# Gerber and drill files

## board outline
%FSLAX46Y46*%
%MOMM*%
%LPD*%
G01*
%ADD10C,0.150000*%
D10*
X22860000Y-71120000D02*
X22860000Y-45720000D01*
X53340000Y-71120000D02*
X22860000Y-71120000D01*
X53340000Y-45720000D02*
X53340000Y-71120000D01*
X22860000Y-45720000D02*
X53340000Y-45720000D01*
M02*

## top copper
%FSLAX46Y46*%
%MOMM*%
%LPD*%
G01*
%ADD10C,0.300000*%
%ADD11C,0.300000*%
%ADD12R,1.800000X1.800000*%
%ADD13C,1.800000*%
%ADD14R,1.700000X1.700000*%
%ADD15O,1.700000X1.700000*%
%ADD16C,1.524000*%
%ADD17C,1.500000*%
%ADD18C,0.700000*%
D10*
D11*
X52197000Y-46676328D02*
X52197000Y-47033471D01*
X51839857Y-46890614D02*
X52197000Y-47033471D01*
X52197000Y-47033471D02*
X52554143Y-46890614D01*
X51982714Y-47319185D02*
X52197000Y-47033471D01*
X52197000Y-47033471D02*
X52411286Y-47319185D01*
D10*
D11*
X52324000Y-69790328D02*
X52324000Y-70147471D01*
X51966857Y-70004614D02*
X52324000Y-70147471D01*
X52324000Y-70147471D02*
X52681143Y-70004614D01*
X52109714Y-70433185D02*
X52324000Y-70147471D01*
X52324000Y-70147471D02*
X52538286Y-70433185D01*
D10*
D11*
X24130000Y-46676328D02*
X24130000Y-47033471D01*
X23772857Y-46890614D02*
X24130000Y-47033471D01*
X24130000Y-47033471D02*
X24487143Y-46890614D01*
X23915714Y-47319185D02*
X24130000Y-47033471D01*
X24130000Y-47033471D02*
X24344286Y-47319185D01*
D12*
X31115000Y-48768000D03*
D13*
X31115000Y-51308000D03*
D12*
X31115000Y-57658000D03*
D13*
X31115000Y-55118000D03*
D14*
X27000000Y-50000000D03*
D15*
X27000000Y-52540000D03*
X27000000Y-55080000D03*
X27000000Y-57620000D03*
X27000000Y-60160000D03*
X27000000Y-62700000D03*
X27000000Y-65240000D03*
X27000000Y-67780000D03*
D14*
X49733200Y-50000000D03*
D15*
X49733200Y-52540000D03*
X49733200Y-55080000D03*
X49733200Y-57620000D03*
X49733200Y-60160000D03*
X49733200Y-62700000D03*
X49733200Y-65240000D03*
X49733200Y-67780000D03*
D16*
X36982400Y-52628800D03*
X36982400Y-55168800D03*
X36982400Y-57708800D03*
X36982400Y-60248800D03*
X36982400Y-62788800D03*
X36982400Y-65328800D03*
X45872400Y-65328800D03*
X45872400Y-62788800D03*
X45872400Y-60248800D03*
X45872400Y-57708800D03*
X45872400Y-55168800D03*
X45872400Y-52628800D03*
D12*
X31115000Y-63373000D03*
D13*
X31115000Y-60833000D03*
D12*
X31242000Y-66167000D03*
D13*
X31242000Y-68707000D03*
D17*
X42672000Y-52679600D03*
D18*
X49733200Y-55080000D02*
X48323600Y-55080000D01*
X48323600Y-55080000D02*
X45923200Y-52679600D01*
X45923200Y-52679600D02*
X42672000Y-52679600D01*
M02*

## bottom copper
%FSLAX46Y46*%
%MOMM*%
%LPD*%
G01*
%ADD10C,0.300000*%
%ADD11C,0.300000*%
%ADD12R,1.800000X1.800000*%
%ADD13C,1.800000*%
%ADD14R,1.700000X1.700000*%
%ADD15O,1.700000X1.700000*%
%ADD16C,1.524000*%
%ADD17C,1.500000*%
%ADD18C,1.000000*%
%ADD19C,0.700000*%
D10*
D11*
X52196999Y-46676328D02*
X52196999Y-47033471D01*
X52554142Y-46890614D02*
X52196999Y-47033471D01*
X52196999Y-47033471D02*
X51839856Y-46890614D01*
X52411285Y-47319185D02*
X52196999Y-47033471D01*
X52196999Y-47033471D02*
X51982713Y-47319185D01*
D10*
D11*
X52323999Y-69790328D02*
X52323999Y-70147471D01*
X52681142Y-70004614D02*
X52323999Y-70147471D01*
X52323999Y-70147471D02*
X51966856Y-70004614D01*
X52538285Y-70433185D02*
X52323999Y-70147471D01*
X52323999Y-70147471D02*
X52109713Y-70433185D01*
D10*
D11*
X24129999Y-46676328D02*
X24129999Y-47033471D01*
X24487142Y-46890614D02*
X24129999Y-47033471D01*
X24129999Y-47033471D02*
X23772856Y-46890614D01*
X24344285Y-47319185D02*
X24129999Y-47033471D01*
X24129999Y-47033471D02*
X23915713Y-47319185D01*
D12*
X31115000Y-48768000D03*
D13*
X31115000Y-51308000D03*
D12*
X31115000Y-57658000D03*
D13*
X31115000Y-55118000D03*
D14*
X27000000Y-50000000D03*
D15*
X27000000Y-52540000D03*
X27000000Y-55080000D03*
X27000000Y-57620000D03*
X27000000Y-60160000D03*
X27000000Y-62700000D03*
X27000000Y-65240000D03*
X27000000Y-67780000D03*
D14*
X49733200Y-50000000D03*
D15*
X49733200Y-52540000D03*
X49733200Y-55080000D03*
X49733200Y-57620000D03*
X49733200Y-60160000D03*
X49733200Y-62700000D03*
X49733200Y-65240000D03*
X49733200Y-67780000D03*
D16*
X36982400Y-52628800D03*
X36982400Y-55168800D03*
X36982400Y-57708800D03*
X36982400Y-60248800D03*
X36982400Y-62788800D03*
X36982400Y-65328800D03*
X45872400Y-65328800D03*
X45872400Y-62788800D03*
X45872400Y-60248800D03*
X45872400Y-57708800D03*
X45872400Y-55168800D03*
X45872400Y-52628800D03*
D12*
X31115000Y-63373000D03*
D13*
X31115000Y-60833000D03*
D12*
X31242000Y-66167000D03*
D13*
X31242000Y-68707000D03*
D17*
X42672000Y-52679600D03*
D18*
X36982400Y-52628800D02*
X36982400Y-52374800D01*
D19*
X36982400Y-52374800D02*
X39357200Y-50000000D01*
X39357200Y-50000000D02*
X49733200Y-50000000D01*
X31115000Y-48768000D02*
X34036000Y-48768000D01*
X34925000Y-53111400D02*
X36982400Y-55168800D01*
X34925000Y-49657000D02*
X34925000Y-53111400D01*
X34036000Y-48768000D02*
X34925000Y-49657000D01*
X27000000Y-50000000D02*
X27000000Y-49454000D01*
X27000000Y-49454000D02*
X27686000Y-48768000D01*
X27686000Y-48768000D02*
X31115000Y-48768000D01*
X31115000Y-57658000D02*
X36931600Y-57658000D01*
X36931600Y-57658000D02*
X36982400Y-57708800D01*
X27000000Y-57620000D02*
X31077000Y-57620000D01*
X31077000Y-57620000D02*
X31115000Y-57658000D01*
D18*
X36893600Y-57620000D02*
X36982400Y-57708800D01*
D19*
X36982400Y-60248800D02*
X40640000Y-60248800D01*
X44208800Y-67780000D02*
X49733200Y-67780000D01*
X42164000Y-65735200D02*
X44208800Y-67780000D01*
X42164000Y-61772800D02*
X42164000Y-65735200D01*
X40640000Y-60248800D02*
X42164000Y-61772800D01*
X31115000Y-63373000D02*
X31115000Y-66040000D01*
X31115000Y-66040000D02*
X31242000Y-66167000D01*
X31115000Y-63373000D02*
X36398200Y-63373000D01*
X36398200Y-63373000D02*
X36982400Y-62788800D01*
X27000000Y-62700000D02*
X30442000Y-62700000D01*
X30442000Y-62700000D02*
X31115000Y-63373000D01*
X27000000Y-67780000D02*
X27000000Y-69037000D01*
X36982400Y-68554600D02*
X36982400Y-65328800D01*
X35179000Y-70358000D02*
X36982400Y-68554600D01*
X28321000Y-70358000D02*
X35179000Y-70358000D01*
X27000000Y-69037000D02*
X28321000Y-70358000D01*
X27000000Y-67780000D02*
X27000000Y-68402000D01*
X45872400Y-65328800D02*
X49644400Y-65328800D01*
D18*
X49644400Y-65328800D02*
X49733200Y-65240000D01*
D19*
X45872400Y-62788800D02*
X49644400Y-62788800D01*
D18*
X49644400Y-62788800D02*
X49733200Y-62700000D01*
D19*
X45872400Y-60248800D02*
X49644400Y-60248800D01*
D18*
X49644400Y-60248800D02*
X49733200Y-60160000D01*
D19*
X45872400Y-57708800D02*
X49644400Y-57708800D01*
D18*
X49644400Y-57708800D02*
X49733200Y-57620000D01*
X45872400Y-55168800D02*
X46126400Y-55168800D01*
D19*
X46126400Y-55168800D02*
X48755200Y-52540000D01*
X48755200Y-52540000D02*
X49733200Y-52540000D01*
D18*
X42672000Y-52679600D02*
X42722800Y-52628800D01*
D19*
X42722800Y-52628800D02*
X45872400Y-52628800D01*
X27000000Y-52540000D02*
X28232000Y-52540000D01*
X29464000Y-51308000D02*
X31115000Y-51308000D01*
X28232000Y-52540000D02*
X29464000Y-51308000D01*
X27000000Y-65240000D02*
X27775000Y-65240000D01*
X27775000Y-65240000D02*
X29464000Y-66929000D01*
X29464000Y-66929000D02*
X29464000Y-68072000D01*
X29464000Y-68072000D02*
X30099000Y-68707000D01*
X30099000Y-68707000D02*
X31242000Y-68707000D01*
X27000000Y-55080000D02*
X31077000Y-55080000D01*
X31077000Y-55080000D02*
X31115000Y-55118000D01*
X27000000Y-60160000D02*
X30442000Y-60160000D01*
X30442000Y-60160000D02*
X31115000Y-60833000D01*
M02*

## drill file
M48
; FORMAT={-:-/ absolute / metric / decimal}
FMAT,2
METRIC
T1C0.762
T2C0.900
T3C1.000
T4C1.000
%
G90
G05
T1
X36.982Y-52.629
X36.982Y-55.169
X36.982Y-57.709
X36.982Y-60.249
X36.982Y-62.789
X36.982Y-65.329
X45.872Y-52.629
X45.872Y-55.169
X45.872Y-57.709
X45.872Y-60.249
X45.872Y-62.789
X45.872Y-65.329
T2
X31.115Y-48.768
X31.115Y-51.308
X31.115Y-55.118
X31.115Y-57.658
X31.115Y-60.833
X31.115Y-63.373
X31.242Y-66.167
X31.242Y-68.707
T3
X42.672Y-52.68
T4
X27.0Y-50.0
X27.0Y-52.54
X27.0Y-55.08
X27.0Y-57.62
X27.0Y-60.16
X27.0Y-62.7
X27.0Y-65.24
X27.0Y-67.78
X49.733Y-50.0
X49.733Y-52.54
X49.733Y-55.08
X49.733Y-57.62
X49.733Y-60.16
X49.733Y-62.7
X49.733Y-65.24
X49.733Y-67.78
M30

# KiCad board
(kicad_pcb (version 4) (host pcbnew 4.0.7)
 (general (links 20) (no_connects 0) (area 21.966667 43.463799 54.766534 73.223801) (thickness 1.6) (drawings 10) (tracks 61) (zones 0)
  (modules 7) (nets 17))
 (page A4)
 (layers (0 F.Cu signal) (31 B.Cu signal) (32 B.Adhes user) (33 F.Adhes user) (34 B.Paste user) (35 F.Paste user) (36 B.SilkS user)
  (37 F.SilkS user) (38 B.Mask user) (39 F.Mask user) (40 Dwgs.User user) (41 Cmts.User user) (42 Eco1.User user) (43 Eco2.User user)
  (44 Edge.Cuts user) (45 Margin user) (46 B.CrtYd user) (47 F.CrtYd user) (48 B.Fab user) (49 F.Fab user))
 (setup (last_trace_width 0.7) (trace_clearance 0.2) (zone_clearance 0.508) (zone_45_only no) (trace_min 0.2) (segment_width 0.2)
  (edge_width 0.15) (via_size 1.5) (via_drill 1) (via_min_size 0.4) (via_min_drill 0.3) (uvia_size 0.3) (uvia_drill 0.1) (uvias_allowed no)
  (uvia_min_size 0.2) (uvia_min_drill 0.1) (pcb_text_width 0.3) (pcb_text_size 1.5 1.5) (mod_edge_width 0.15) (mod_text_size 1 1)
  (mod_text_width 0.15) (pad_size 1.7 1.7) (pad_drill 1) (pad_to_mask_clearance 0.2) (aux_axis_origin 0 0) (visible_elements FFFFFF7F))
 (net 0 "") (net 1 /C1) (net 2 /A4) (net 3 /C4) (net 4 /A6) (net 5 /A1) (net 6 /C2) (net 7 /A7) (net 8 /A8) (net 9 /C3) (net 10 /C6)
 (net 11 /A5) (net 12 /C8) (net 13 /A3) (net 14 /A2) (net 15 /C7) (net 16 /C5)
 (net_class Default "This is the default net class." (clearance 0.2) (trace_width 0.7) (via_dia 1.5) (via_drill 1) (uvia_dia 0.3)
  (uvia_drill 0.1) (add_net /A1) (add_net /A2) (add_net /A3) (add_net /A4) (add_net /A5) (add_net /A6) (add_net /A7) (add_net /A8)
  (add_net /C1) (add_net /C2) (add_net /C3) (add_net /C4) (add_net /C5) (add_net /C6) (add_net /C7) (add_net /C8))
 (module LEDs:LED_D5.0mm (layer F.Cu) (at 31.115 48.768 270)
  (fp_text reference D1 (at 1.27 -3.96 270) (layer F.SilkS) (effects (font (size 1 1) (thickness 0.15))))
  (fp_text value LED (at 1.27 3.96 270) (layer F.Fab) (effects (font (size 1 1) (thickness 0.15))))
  (pad 1 thru_hole rect (at 0 0 270) (size 1.8 1.8) (drill 0.9) (layers *.Cu *.Mask) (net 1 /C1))
  (pad 2 thru_hole circle (at 2.54 0 270) (size 1.8 1.8) (drill 0.9) (layers *.Cu *.Mask) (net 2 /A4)))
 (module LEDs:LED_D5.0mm (layer F.Cu) (at 31.115 57.658 90)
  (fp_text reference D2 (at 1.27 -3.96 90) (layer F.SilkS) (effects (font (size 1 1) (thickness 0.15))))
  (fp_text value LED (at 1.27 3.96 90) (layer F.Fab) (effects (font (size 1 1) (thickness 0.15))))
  (pad 1 thru_hole rect (at 0 0 90) (size 1.8 1.8) (drill 0.9) (layers *.Cu *.Mask) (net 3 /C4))
  (pad 2 thru_hole circle (at 2.54 0 90) (size 1.8 1.8) (drill 0.9) (layers *.Cu *.Mask) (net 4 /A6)))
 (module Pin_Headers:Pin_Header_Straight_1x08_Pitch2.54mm (layer F.Cu) (at 27 50)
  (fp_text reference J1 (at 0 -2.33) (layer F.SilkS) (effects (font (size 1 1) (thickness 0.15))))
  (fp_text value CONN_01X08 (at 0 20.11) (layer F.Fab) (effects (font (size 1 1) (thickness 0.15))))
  (pad 1 thru_hole rect (at 0 0) (size 1.7 1.7) (drill 1) (layers *.Cu *.Mask) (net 1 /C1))
  (pad 2 thru_hole oval (at 0 2.54) (size 1.7 1.7) (drill 1) (layers *.Cu *.Mask) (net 2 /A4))
  (pad 3 thru_hole oval (at 0 5.08) (size 1.7 1.7) (drill 1) (layers *.Cu *.Mask) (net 4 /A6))
  (pad 4 thru_hole oval (at 0 7.62) (size 1.7 1.7) (drill 1) (layers *.Cu *.Mask) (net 3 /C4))
  (pad 5 thru_hole oval (at 0 10.16) (size 1.7 1.7) (drill 1) (layers *.Cu *.Mask) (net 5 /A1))
  (pad 6 thru_hole oval (at 0 12.7) (size 1.7 1.7) (drill 1) (layers *.Cu *.Mask) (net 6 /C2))
  (pad 7 thru_hole oval (at 0 15.24) (size 1.7 1.7) (drill 1) (layers *.Cu *.Mask) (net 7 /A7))
  (pad 8 thru_hole oval (at 0 17.78) (size 1.7 1.7) (drill 1) (layers *.Cu *.Mask) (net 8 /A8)))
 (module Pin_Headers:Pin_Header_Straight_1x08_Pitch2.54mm (layer F.Cu) (at 49.7332 50)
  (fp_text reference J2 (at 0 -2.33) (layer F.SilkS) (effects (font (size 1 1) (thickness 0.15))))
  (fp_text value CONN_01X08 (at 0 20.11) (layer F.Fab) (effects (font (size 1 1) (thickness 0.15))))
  (pad 1 thru_hole rect (at 0 0) (size 1.7 1.7) (drill 1) (layers *.Cu *.Mask) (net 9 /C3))
  (pad 2 thru_hole oval (at 0 2.54) (size 1.7 1.7) (drill 1) (layers *.Cu *.Mask) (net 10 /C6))
  (pad 3 thru_hole oval (at 0 5.08) (size 1.7 1.7) (drill 1) (layers *.Cu *.Mask) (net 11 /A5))
  (pad 4 thru_hole oval (at 0 7.62) (size 1.7 1.7) (drill 1) (layers *.Cu *.Mask) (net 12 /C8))
  (pad 5 thru_hole oval (at 0 10.16) (size 1.7 1.7) (drill 1) (layers *.Cu *.Mask) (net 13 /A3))
  (pad 6 thru_hole oval (at 0 12.7) (size 1.7 1.7) (drill 1) (layers *.Cu *.Mask) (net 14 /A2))
  (pad 7 thru_hole oval (at 0 15.24) (size 1.7 1.7) (drill 1) (layers *.Cu *.Mask) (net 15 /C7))
  (pad 8 thru_hole oval (at 0 17.78) (size 1.7 1.7) (drill 1) (layers *.Cu *.Mask) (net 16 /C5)))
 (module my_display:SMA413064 (layer F.Cu) (at 36.9824 52.6288)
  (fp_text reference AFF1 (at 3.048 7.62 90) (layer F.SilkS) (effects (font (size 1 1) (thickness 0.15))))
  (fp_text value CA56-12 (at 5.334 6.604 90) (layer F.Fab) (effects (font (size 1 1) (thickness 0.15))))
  (pad 1 thru_hole circle (at 0 0) (size 1.524 1.524) (drill 0.762) (layers *.Cu *.Mask) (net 9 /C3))
  (pad 2 thru_hole circle (at 0 2.54) (size 1.524 1.524) (drill 0.762) (layers *.Cu *.Mask) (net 1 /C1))
  (pad 3 thru_hole circle (at 0 5.08) (size 1.524 1.524) (drill 0.762) (layers *.Cu *.Mask) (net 3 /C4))
  (pad 4 thru_hole circle (at 0 7.62) (size 1.524 1.524) (drill 0.762) (layers *.Cu *.Mask) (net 16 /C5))
  (pad 5 thru_hole circle (at 0 10.16) (size 1.524 1.524) (drill 0.762) (layers *.Cu *.Mask) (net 6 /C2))
  (pad 6 thru_hole circle (at 0 12.7) (size 1.524 1.524) (drill 0.762) (layers *.Cu *.Mask) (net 8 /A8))
  (pad 7 thru_hole circle (at 8.89 12.7) (size 1.524 1.524) (drill 0.762) (layers *.Cu *.Mask) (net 15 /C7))
  (pad 8 thru_hole circle (at 8.89 10.16) (size 1.524 1.524) (drill 0.762) (layers *.Cu *.Mask) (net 14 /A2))
  (pad 9 thru_hole circle (at 8.89 7.62) (size 1.524 1.524) (drill 0.762) (layers *.Cu *.Mask) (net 13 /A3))
  (pad 10 thru_hole circle (at 8.89 5.08) (size 1.524 1.524) (drill 0.762) (layers *.Cu *.Mask) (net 12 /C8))
  (pad 11 thru_hole circle (at 8.89 2.54) (size 1.524 1.524) (drill 0.762) (layers *.Cu *.Mask) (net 10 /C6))
  (pad 12 thru_hole circle (at 8.89 0) (size 1.524 1.524) (drill 0.762) (layers *.Cu *.Mask) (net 11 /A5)))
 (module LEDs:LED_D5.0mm (layer F.Cu) (at 31.115 63.373 90)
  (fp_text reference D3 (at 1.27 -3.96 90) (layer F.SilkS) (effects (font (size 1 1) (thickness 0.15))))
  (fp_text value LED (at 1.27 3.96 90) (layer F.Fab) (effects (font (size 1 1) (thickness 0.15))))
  (pad 1 thru_hole rect (at 0 0 90) (size 1.8 1.8) (drill 0.9) (layers *.Cu *.Mask) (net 6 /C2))
  (pad 2 thru_hole circle (at 2.54 0 90) (size 1.8 1.8) (drill 0.9) (layers *.Cu *.Mask) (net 5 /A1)))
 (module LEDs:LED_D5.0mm (layer F.Cu) (at 31.242 66.167 270)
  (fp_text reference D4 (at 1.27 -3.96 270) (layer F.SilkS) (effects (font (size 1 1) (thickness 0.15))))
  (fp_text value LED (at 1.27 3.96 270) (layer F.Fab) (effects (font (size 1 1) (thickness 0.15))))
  (pad 1 thru_hole rect (at 0 0 270) (size 1.8 1.8) (drill 0.9) (layers *.Cu *.Mask) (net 6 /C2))
  (pad 2 thru_hole circle (at 2.54 0 270) (size 1.8 1.8) (drill 0.9) (layers *.Cu *.Mask) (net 7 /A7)))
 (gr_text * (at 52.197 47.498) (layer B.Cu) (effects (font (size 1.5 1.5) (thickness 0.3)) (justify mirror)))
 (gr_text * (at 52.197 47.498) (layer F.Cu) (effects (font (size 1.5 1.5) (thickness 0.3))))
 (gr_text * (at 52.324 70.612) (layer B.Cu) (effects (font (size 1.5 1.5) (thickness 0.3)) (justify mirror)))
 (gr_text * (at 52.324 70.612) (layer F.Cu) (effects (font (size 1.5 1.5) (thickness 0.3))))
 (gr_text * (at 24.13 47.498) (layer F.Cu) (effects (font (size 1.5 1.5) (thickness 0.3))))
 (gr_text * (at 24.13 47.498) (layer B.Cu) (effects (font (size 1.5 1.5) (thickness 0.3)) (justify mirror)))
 (gr_line (start 22.86 71.12) (end 22.86 45.72) (angle 90) (layer Edge.Cuts) (width 0.15))
 (gr_line (start 53.34 71.12) (end 22.86 71.12) (angle 90) (layer Edge.Cuts) (width 0.15))
 (gr_line (start 53.34 45.72) (end 53.34 71.12) (angle 90) (layer Edge.Cuts) (width 0.15))
 (gr_line (start 22.86 45.72) (end 53.34 45.72) (angle 90) (layer Edge.Cuts) (width 0.15))
 (segment (start 36.9824 52.6288) (end 36.9824 52.3748) (width 1) (layer B.Cu) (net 9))
 (segment (start 36.9824 52.3748) (end 39.3572 50) (width 0.7) (layer B.Cu) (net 9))
 (segment (start 39.3572 50) (end 49.7332 50) (width 0.7) (layer B.Cu) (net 9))
 (segment (start 31.115 48.768) (end 34.036 48.768) (width 0.7) (layer B.Cu) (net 1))
 (segment (start 34.925 53.1114) (end 36.9824 55.1688) (width 0.7) (layer B.Cu) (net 1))
 (segment (start 34.925 49.657) (end 34.925 53.1114) (width 0.7) (layer B.Cu) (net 1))
 (segment (start 34.036 48.768) (end 34.925 49.657) (width 0.7) (layer B.Cu) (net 1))
 (segment (start 27 50) (end 27 49.454) (width 0.7) (layer B.Cu) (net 1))
 (segment (start 27 49.454) (end 27.686 48.768) (width 0.7) (layer B.Cu) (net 1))
 (segment (start 27.686 48.768) (end 31.115 48.768) (width 0.7) (layer B.Cu) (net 1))
 (segment (start 31.115 57.658) (end 36.9316 57.658) (width 0.7) (layer B.Cu) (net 3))
 (segment (start 36.9316 57.658) (end 36.9824 57.7088) (width 0.7) (layer B.Cu) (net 3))
 (segment (start 27 57.62) (end 31.077 57.62) (width 0.7) (layer B.Cu) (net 3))
 (segment (start 31.077 57.62) (end 31.115 57.658) (width 0.7) (layer B.Cu) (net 3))
 (segment (start 36.8936 57.62) (end 36.9824 57.7088) (width 1) (layer B.Cu) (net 3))
 (segment (start 36.9824 60.2488) (end 40.64 60.2488) (width 0.7) (layer B.Cu) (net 16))
 (segment (start 44.2088 67.78) (end 49.7332 67.78) (width 0.7) (layer B.Cu) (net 16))
 (segment (start 42.164 65.7352) (end 44.2088 67.78) (width 0.7) (layer B.Cu) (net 16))
 (segment (start 42.164 61.7728) (end 42.164 65.7352) (width 0.7) (layer B.Cu) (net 16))
 (segment (start 40.64 60.2488) (end 42.164 61.7728) (width 0.7) (layer B.Cu) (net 16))
 (segment (start 31.115 63.373) (end 31.115 66.04) (width 0.7) (layer B.Cu) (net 6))
 (segment (start 31.115 66.04) (end 31.242 66.167) (width 0.7) (layer B.Cu) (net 6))
 (segment (start 31.115 63.373) (end 36.3982 63.373) (width 0.7) (layer B.Cu) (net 6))
 (segment (start 36.3982 63.373) (end 36.9824 62.7888) (width 0.7) (layer B.Cu) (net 6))
 (segment (start 27 62.7) (end 30.442 62.7) (width 0.7) (layer B.Cu) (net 6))
 (segment (start 30.442 62.7) (end 31.115 63.373) (width 0.7) (layer B.Cu) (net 6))
 (segment (start 27 67.78) (end 27 69.037) (width 0.7) (layer B.Cu) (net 8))
 (segment (start 36.9824 68.5546) (end 36.9824 65.3288) (width 0.7) (layer B.Cu) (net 8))
 (segment (start 35.179 70.358) (end 36.9824 68.5546) (width 0.7) (layer B.Cu) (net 8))
 (segment (start 28.321 70.358) (end 35.179 70.358) (width 0.7) (layer B.Cu) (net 8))
 (segment (start 27 69.037) (end 28.321 70.358) (width 0.7) (layer B.Cu) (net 8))
 (segment (start 27 67.78) (end 27 68.402) (width 0.7) (layer B.Cu) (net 8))
 (segment (start 45.8724 65.3288) (end 49.6444 65.3288) (width 0.7) (layer B.Cu) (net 15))
 (segment (start 49.6444 65.3288) (end 49.7332 65.24) (width 1) (layer B.Cu) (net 15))
 (segment (start 45.8724 62.7888) (end 49.6444 62.7888) (width 0.7) (layer B.Cu) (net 14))
 (segment (start 49.6444 62.7888) (end 49.7332 62.7) (width 1) (layer B.Cu) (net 14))
 (segment (start 45.8724 60.2488) (end 49.6444 60.2488) (width 0.7) (layer B.Cu) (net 13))
 (segment (start 49.6444 60.2488) (end 49.7332 60.16) (width 1) (layer B.Cu) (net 13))
 (segment (start 45.8724 57.7088) (end 49.6444 57.7088) (width 0.7) (layer B.Cu) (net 12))
 (segment (start 49.6444 57.7088) (end 49.7332 57.62) (width 1) (layer B.Cu) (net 12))
 (segment (start 45.8724 55.1688) (end 46.1264 55.1688) (width 1) (layer B.Cu) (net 10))
 (segment (start 46.1264 55.1688) (end 48.7552 52.54) (width 0.7) (layer B.Cu) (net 10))
 (segment (start 48.7552 52.54) (end 49.7332 52.54) (width 0.7) (layer B.Cu) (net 10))
 (segment (start 49.7332 55.08) (end 48.3236 55.08) (width 0.7) (layer F.Cu) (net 11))
 (segment (start 48.3236 55.08) (end 45.9232 52.6796) (width 0.7) (layer F.Cu) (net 11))
 (segment (start 45.9232 52.6796) (end 42.672 52.6796) (width 0.7) (layer F.Cu) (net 11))
 (via (at 42.672 52.6796) (size 1.5) (drill 1) (layers F.Cu B.Cu) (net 11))
 (segment (start 42.672 52.6796) (end 42.7228 52.6288) (width 1) (layer B.Cu) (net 11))
 (segment (start 42.7228 52.6288) (end 45.8724 52.6288) (width 0.7) (layer B.Cu) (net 11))
 (segment (start 27 52.54) (end 28.232 52.54) (width 0.7) (layer B.Cu) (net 2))
 (segment (start 29.464 51.308) (end 31.115 51.308) (width 0.7) (layer B.Cu) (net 2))
 (segment (start 28.232 52.54) (end 29.464 51.308) (width 0.7) (layer B.Cu) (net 2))
 (segment (start 27 65.24) (end 27.775 65.24) (width 0.7) (layer B.Cu) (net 7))
 (segment (start 27.775 65.24) (end 29.464 66.929) (width 0.7) (layer B.Cu) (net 7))
 (segment (start 29.464 66.929) (end 29.464 68.072) (width 0.7) (layer B.Cu) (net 7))
 (segment (start 29.464 68.072) (end 30.099 68.707) (width 0.7) (layer B.Cu) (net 7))
 (segment (start 30.099 68.707) (end 31.242 68.707) (width 0.7) (layer B.Cu) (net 7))
 (segment (start 27 55.08) (end 31.077 55.08) (width 0.7) (layer B.Cu) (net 4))
 (segment (start 31.077 55.08) (end 31.115 55.118) (width 0.7) (layer B.Cu) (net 4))
 (segment (start 27 60.16) (end 30.442 60.16) (width 0.7) (layer B.Cu) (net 5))
 (segment (start 30.442 60.16) (end 31.115 60.833) (width 0.7) (layer B.Cu) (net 5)))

